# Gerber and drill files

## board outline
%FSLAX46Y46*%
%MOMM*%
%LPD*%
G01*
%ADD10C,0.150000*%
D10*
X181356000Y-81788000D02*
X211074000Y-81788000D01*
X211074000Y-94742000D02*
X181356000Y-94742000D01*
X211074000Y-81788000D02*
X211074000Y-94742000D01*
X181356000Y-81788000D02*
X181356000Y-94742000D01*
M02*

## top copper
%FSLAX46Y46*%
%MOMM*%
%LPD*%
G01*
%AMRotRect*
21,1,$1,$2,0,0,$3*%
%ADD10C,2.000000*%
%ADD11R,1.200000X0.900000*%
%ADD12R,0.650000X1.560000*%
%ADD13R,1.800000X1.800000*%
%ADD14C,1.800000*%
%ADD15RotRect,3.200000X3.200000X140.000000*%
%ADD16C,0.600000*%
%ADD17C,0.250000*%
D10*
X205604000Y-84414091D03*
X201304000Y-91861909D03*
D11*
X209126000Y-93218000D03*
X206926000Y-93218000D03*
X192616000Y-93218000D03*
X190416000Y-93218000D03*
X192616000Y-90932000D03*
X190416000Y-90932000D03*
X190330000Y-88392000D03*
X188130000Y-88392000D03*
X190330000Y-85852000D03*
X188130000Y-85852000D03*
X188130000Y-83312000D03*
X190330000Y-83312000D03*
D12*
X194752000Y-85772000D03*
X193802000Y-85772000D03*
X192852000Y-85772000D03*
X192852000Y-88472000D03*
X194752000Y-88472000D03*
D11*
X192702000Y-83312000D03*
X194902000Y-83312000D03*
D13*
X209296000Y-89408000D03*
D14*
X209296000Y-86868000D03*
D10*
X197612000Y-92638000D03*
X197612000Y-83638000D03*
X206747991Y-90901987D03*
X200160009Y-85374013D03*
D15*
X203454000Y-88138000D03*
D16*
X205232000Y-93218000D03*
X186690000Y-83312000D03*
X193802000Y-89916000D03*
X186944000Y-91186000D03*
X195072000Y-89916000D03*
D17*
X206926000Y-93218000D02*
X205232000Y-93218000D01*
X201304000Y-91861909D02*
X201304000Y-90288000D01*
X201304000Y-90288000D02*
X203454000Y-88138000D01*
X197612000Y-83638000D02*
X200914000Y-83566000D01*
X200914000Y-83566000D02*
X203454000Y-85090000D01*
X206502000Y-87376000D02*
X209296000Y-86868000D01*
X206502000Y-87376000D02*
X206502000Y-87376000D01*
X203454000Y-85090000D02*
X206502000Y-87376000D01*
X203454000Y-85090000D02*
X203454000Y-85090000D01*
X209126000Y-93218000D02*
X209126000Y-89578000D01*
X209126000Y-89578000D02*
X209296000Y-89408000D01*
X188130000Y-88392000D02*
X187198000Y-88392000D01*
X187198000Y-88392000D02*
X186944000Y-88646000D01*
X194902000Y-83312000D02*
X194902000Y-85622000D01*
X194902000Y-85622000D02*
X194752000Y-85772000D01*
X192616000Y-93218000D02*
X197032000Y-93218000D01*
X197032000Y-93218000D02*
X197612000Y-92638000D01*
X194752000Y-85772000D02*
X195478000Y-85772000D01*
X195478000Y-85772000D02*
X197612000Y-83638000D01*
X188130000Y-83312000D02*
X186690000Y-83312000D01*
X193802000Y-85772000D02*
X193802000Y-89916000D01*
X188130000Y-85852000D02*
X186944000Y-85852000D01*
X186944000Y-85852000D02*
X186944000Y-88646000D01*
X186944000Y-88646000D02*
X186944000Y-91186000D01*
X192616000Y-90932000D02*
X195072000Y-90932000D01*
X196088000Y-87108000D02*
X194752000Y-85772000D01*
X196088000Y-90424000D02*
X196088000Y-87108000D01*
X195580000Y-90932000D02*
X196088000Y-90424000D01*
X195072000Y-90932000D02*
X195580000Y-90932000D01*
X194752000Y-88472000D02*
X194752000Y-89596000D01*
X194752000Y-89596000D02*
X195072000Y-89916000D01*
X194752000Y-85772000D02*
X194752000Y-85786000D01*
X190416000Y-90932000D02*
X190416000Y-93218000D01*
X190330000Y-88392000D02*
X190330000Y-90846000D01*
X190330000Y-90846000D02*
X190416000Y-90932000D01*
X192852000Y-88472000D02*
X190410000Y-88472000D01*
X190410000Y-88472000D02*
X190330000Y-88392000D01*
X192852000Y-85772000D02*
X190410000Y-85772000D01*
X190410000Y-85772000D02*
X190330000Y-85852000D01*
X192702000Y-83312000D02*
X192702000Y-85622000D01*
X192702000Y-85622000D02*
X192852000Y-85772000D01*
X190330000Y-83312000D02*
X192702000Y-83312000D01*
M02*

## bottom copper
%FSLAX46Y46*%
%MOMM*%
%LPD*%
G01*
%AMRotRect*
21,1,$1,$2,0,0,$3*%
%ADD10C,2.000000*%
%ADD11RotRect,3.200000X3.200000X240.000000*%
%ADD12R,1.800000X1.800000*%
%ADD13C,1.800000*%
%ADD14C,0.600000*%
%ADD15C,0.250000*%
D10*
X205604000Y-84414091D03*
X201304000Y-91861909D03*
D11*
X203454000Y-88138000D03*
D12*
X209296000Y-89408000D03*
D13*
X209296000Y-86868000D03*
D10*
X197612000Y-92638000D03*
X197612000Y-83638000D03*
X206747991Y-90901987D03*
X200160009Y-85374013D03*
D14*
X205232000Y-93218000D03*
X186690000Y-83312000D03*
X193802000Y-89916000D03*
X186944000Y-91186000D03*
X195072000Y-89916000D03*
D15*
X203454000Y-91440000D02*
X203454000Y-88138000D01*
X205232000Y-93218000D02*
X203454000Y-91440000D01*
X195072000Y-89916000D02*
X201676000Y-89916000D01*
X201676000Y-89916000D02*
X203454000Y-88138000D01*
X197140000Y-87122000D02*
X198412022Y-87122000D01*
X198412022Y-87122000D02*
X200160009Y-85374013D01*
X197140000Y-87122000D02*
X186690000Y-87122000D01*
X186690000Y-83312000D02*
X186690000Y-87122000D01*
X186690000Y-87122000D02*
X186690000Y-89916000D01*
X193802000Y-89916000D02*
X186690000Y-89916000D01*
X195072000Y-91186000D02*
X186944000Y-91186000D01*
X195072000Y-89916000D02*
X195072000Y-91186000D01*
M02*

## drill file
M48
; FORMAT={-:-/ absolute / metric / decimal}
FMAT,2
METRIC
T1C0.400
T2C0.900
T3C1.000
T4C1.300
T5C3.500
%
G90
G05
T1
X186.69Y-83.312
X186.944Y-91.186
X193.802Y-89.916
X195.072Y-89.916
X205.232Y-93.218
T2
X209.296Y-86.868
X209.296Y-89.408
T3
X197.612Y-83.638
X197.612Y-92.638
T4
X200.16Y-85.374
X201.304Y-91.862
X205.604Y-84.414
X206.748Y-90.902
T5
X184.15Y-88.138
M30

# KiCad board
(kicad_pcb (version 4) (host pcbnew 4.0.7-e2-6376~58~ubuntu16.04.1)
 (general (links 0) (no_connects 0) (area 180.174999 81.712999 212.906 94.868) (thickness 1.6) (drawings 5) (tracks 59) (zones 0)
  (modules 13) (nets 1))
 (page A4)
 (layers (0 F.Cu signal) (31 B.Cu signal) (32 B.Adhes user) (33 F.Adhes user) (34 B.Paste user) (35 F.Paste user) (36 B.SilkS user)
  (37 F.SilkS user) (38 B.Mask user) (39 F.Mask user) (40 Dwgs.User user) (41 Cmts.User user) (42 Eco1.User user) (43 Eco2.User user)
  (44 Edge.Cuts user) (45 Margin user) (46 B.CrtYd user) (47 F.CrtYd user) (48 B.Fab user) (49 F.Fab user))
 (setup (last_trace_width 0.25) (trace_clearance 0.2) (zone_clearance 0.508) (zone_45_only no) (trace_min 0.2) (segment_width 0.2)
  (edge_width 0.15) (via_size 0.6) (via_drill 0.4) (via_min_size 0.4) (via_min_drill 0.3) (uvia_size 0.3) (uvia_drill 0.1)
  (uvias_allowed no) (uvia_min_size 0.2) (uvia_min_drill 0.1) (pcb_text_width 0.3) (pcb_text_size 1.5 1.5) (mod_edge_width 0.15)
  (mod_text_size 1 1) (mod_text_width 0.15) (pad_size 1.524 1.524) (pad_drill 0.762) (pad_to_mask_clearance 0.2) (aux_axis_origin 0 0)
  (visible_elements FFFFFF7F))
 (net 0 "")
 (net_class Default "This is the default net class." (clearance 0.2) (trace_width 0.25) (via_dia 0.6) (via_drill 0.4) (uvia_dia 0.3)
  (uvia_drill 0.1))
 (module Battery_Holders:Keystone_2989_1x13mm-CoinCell (layer B.Cu) (at 203.454 88.138 240)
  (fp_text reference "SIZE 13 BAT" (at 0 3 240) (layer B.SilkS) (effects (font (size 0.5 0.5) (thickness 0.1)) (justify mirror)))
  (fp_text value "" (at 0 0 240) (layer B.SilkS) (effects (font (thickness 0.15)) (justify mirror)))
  (pad 1 thru_hole circle (at -4.3 0 240) (size 2 2) (drill 1.3) (layers *.Cu *.Mask))
  (pad 1 thru_hole circle (at 4.3 0 240) (size 2 2) (drill 1.3) (layers *.Cu *.Mask))
  (pad 2 smd rect (at 0 0 240) (size 3.2 3.2) (layers B.Cu B.Mask)))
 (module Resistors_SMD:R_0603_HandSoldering (layer F.Cu) (at 208.026 93.218 180)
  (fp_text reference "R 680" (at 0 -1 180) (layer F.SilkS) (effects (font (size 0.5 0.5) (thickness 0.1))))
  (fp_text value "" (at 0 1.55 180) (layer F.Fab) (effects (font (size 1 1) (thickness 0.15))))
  (pad 1 smd rect (at -1.1 0 180) (size 1.2 0.9) (layers F.Cu F.Paste F.Mask))
  (pad 2 smd rect (at 1.1 0 180) (size 1.2 0.9) (layers F.Cu F.Paste F.Mask)))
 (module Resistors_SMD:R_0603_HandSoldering (layer F.Cu) (at 191.516 93.218 180)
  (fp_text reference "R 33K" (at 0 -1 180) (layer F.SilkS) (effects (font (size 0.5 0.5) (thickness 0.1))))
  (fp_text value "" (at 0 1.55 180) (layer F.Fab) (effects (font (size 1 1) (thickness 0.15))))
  (pad 1 smd rect (at -1.1 0 180) (size 1.2 0.9) (layers F.Cu F.Paste F.Mask))
  (pad 2 smd rect (at 1.1 0 180) (size 1.2 0.9) (layers F.Cu F.Paste F.Mask)))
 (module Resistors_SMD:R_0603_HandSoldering (layer F.Cu) (at 191.516 90.932 180)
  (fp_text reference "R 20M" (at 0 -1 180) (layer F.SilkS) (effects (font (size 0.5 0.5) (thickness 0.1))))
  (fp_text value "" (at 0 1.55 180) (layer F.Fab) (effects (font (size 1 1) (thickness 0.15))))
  (pad 1 smd rect (at -1.1 0 180) (size 1.2 0.9) (layers F.Cu F.Paste F.Mask))
  (pad 2 smd rect (at 1.1 0 180) (size 1.2 0.9) (layers F.Cu F.Paste F.Mask)))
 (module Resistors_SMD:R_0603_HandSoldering (layer F.Cu) (at 189.23 88.392 180)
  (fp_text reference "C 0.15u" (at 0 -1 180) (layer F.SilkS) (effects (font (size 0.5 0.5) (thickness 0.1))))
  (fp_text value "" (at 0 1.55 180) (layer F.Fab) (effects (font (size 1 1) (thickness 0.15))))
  (pad 1 smd rect (at -1.1 0 180) (size 1.2 0.9) (layers F.Cu F.Paste F.Mask))
  (pad 2 smd rect (at 1.1 0 180) (size 1.2 0.9) (layers F.Cu F.Paste F.Mask)))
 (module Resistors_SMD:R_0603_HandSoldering (layer F.Cu) (at 189.23 85.852 180)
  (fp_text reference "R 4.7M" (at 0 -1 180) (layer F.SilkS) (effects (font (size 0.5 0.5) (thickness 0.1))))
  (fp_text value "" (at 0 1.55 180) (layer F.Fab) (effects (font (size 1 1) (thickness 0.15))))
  (pad 1 smd rect (at -1.1 0 180) (size 1.2 0.9) (layers F.Cu F.Paste F.Mask))
  (pad 2 smd rect (at 1.1 0 180) (size 1.2 0.9) (layers F.Cu F.Paste F.Mask)))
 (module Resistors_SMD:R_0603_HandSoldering (layer F.Cu) (at 189.23 83.312)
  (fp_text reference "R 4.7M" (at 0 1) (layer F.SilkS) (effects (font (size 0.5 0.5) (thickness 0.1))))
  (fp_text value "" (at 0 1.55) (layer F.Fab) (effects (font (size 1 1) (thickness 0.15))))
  (pad 1 smd rect (at -1.1 0) (size 1.2 0.9) (layers F.Cu F.Paste F.Mask))
  (pad 2 smd rect (at 1.1 0) (size 1.2 0.9) (layers F.Cu F.Paste F.Mask)))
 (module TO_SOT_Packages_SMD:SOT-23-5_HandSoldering (layer F.Cu) (at 193.802 87.122 270)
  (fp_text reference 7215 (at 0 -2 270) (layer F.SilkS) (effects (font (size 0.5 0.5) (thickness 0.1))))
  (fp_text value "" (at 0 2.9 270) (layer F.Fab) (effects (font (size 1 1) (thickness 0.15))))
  (pad 1 smd rect (at -1.35 -0.95 270) (size 1.56 0.65) (layers F.Cu F.Paste F.Mask))
  (pad 2 smd rect (at -1.35 0 270) (size 1.56 0.65) (layers F.Cu F.Paste F.Mask))
  (pad 3 smd rect (at -1.35 0.95 270) (size 1.56 0.65) (layers F.Cu F.Paste F.Mask))
  (pad 4 smd rect (at 1.35 0.95 270) (size 1.56 0.65) (layers F.Cu F.Paste F.Mask))
  (pad 5 smd rect (at 1.35 -0.95 270) (size 1.56 0.65) (layers F.Cu F.Paste F.Mask)))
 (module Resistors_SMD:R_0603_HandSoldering (layer F.Cu) (at 193.802 83.312)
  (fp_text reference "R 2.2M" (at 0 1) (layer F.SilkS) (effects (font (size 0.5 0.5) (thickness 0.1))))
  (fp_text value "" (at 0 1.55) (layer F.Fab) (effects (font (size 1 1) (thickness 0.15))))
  (pad 1 smd rect (at -1.1 0) (size 1.2 0.9) (layers F.Cu F.Paste F.Mask))
  (pad 2 smd rect (at 1.1 0) (size 1.2 0.9) (layers F.Cu F.Paste F.Mask)))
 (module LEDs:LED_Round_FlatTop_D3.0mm (layer F.Cu) (at 209.296 89.408 90)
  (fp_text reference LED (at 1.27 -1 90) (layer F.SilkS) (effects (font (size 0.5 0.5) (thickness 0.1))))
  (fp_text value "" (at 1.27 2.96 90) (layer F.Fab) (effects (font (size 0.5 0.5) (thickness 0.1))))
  (pad 1 thru_hole rect (at 0 0 90) (size 1.8 1.8) (drill 0.9) (layers *.Cu *.Mask))
  (pad 2 thru_hole circle (at 2.54 0 90) (size 1.8 1.8) (drill 0.9) (layers *.Cu *.Mask)))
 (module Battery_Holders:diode (layer F.Cu) (at 197.612 88.138 90)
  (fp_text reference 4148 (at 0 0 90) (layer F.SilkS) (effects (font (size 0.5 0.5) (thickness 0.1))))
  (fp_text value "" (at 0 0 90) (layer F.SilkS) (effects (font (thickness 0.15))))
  (pad 1 thru_hole circle (at -4.5 0 90) (size 2 2) (drill 1) (layers *.Cu *.Mask))
  (pad 2 thru_hole circle (at 4.5 0 90) (size 2 2) (drill 1) (layers *.Cu *.Mask)))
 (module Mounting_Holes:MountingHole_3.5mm (layer F.Cu) (at 184.15 88.138)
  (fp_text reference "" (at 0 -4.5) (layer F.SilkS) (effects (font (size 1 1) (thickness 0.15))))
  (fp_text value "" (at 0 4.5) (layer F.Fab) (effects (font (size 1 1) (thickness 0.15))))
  (pad 1 np_thru_hole circle (at 0 0) (size 3.5 3.5) (drill 3.5) (layers *.Cu *.Mask)))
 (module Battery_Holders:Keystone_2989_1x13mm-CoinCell (layer F.Cu) (at 203.454 88.138 140)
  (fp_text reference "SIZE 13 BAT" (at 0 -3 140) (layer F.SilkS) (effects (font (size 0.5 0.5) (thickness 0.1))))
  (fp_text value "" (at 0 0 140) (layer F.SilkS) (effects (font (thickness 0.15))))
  (pad 1 thru_hole circle (at -4.3 0 140) (size 2 2) (drill 1.3) (layers *.Cu *.Mask))
  (pad 1 thru_hole circle (at 4.3 0 140) (size 2 2) (drill 1.3) (layers *.Cu *.Mask))
  (pad 2 smd rect (at 0 0 140) (size 3.2 3.2) (layers F.Cu F.Mask)))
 (gr_line (start 181.356 81.788) (end 211.074 81.788) (angle 90) (layer Edge.Cuts) (width 0.15))
 (gr_line (start 211.074 94.742) (end 181.356 94.742) (angle 90) (layer Edge.Cuts) (width 0.15))
 (gr_line (start 211.074 81.788) (end 211.074 94.742) (angle 90) (layer Edge.Cuts) (width 0.15))
 (gr_line (start 181.356 81.788) (end 181.356 94.742) (angle 90) (layer Edge.Cuts) (width 0.15))
 (segment (start 206.926 93.218) (end 205.232 93.218) (width 0.25) (layer F.Cu) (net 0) (status 400000))
 (segment (start 203.454 91.44) (end 203.454 88.138) (width 0.25) (layer B.Cu) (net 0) (status 800000))
 (segment (start 205.232 93.218) (end 203.454 91.44) (width 0.25) (layer B.Cu) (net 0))
 (via (at 205.232 93.218) (size 0.6) (drill 0.4) (layers F.Cu B.Cu) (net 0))
 (segment (start 195.072 89.916) (end 201.676 89.916) (width 0.25) (layer B.Cu) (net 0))
 (segment (start 201.676 89.916) (end 203.454 88.138) (width 0.25) (layer B.Cu) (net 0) (status 800000))
 (segment (start 201.304 91.861909) (end 201.304 90.288) (width 0.25) (layer F.Cu) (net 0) (status 400000))
 (segment (start 201.304 90.288) (end 203.454 88.138) (width 0.25) (layer F.Cu) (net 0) (status 800000))
 (segment (start 197.14 87.122) (end 198.412022 87.122) (width 0.25) (layer B.Cu) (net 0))
 (segment (start 198.412022 87.122) (end 200.160009 85.374013) (width 0.25) (layer B.Cu) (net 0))
 (segment (start 197.14 87.122) (end 186.69 87.122) (width 0.25) (layer B.Cu) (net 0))
 (segment (start 197.612 83.638) (end 200.914 83.566) (width 0.25) (layer F.Cu) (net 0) (status 400000))
 (segment (start 200.914 83.566) (end 203.454 85.09) (width 0.25) (layer F.Cu) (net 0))
 (segment (start 206.502 87.376) (end 209.296 86.868) (width 0.25) (layer F.Cu) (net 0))
 (segment (start 206.502 87.376) (end 206.502 87.376) (width 0.25) (layer F.Cu) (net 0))
 (segment (start 203.454 85.09) (end 206.502 87.376) (width 0.25) (layer F.Cu) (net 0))
 (segment (start 203.454 85.09) (end 203.454 85.09) (width 0.25) (layer F.Cu) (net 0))
 (segment (start 209.126 93.218) (end 209.126 89.578) (width 0.25) (layer F.Cu) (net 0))
 (segment (start 209.126 89.578) (end 209.296 89.408) (width 0.25) (layer F.Cu) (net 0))
 (segment (start 188.13 88.392) (end 187.198 88.392) (width 0.25) (layer F.Cu) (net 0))
 (segment (start 187.198 88.392) (end 186.944 88.646) (width 0.25) (layer F.Cu) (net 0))
 (segment (start 194.902 83.312) (end 194.902 85.622) (width 0.25) (layer F.Cu) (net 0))
 (segment (start 194.902 85.622) (end 194.752 85.772) (width 0.25) (layer F.Cu) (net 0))
 (segment (start 192.616 93.218) (end 197.032 93.218) (width 0.25) (layer F.Cu) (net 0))
 (segment (start 197.032 93.218) (end 197.612 92.638) (width 0.25) (layer F.Cu) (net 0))
 (segment (start 194.752 85.772) (end 195.478 85.772) (width 0.25) (layer F.Cu) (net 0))
 (segment (start 195.478 85.772) (end 197.612 83.638) (width 0.25) (layer F.Cu) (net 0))
 (segment (start 188.13 83.312) (end 186.69 83.312) (width 0.25) (layer F.Cu) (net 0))
 (via (at 186.69 83.312) (size 0.6) (drill 0.4) (layers F.Cu B.Cu) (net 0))
 (segment (start 186.69 83.312) (end 186.69 87.122) (width 0.25) (layer B.Cu) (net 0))
 (segment (start 186.69 87.122) (end 186.69 89.916) (width 0.25) (layer B.Cu) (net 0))
 (via (at 193.802 89.916) (size 0.6) (drill 0.4) (layers F.Cu B.Cu) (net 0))
 (segment (start 193.802 89.916) (end 186.69 89.916) (width 0.25) (layer B.Cu) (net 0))
 (segment (start 193.802 85.772) (end 193.802 89.916) (width 0.25) (layer F.Cu) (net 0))
 (segment (start 188.13 85.852) (end 186.944 85.852) (width 0.25) (layer F.Cu) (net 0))
 (via (at 186.944 91.186) (size 0.6) (drill 0.4) (layers F.Cu B.Cu) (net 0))
 (segment (start 186.944 85.852) (end 186.944 88.646) (width 0.25) (layer F.Cu) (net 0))
 (segment (start 186.944 88.646) (end 186.944 91.186) (width 0.25) (layer F.Cu) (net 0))
 (segment (start 192.616 90.932) (end 195.072 90.932) (width 0.25) (layer F.Cu) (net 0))
 (segment (start 196.088 87.108) (end 194.752 85.772) (width 0.25) (layer F.Cu) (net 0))
 (segment (start 196.088 90.424) (end 196.088 87.108) (width 0.25) (layer F.Cu) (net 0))
 (segment (start 195.58 90.932) (end 196.088 90.424) (width 0.25) (layer F.Cu) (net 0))
 (segment (start 195.072 90.932) (end 195.58 90.932) (width 0.25) (layer F.Cu) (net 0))
 (segment (start 194.752 88.472) (end 194.752 89.596) (width 0.25) (layer F.Cu) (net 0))
 (segment (start 195.072 91.186) (end 186.944 91.186) (width 0.25) (layer B.Cu) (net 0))
 (segment (start 195.072 89.916) (end 195.072 91.186) (width 0.25) (layer B.Cu) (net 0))
 (via (at 195.072 89.916) (size 0.6) (drill 0.4) (layers F.Cu B.Cu) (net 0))
 (segment (start 194.752 89.596) (end 195.072 89.916) (width 0.25) (layer F.Cu) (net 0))
 (segment (start 194.752 85.772) (end 194.752 85.786) (width 0.25) (layer F.Cu) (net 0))
 (segment (start 190.416 90.932) (end 190.416 93.218) (width 0.25) (layer F.Cu) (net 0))
 (segment (start 190.33 88.392) (end 190.33 90.846) (width 0.25) (layer F.Cu) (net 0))
 (segment (start 190.33 90.846) (end 190.416 90.932) (width 0.25) (layer F.Cu) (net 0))
 (segment (start 192.852 88.472) (end 190.41 88.472) (width 0.25) (layer F.Cu) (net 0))
 (segment (start 190.41 88.472) (end 190.33 88.392) (width 0.25) (layer F.Cu) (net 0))
 (segment (start 192.852 85.772) (end 190.41 85.772) (width 0.25) (layer F.Cu) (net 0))
 (segment (start 190.41 85.772) (end 190.33 85.852) (width 0.25) (layer F.Cu) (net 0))
 (segment (start 192.702 83.312) (end 192.702 85.622) (width 0.25) (layer F.Cu) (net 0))
 (segment (start 192.702 85.622) (end 192.852 85.772) (width 0.25) (layer F.Cu) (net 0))
 (segment (start 190.33 83.312) (end 192.702 83.312) (width 0.25) (layer F.Cu) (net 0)))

